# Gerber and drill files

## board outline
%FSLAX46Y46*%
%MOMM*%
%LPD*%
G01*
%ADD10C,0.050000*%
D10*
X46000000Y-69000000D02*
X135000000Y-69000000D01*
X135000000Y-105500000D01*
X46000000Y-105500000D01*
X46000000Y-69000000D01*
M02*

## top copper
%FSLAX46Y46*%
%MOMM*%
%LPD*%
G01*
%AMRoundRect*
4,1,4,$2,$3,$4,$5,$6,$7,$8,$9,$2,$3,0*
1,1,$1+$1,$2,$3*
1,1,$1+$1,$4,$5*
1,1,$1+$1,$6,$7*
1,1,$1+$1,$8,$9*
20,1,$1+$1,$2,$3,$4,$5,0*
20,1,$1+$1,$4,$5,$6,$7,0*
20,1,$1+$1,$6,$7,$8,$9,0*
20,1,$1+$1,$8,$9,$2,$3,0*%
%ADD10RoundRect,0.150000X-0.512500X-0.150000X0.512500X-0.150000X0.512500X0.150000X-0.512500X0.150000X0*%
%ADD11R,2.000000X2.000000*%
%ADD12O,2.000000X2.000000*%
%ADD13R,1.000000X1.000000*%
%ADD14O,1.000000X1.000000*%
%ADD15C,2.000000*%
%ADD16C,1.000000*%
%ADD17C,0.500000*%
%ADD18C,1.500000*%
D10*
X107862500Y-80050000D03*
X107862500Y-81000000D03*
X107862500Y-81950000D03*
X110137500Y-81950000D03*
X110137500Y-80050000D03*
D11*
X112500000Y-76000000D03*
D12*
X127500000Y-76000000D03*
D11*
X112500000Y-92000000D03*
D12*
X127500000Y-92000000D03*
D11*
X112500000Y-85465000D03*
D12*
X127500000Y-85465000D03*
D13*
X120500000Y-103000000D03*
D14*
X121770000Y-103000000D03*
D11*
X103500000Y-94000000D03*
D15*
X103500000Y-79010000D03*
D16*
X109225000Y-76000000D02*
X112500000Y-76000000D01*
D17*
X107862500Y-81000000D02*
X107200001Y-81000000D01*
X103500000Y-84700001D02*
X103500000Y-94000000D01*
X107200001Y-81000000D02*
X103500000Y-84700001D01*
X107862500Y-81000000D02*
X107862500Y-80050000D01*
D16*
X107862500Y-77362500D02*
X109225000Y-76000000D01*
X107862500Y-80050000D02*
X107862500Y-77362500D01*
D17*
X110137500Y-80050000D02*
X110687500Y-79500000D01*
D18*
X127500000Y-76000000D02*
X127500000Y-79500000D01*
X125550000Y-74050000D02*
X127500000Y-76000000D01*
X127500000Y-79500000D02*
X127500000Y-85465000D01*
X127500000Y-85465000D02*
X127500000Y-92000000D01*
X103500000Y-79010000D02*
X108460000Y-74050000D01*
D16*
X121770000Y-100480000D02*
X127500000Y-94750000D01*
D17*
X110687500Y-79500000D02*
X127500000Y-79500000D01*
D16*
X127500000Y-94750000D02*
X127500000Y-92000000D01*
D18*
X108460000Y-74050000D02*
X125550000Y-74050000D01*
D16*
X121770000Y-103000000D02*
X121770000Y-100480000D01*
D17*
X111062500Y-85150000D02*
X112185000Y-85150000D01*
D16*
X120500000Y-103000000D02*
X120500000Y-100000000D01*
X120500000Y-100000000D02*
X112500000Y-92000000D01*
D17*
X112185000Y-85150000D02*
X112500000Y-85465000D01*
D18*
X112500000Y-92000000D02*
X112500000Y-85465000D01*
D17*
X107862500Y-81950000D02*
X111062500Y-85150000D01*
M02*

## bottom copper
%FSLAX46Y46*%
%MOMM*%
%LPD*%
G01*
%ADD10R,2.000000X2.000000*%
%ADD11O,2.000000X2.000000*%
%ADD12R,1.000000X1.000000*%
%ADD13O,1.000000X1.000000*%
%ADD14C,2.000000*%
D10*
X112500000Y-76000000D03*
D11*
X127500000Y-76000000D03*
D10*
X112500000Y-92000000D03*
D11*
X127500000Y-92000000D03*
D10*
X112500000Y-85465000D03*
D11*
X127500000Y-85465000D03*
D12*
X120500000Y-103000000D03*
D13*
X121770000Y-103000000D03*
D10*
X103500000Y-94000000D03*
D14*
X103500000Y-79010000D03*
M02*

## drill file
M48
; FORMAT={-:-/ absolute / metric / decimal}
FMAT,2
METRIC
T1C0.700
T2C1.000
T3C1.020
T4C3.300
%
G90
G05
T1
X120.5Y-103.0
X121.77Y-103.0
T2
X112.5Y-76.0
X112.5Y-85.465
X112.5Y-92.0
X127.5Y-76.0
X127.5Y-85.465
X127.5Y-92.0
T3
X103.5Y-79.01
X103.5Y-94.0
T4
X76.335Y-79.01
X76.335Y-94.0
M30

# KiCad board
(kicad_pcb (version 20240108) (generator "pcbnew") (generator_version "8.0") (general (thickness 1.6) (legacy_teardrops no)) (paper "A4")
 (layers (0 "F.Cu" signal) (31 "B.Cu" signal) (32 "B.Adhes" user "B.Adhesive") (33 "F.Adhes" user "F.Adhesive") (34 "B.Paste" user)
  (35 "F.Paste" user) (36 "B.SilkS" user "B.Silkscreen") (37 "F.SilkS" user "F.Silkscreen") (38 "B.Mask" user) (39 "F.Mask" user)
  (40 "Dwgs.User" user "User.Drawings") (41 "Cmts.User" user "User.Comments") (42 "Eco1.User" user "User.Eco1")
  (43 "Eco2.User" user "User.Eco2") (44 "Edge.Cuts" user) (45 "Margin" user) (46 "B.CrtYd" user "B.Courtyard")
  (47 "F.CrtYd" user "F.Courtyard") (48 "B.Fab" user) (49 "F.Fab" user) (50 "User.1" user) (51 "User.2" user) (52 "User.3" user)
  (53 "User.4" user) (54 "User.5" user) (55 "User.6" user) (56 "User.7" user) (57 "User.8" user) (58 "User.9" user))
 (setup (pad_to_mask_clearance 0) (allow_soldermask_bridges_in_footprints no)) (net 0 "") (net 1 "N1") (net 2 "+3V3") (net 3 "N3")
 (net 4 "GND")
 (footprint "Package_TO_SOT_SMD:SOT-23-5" (layer "F.Cu") (at 109 81)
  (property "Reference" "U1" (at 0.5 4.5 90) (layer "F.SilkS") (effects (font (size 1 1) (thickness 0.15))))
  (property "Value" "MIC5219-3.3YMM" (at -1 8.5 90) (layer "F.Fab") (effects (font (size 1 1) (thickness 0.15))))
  (pad "1" smd roundrect (at -1.1375 -0.95) (size 1.325 0.6) (layers "F.Cu" "F.Paste" "F.Mask") (roundrect_rratio 0.25) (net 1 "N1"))
  (pad "2" smd roundrect (at -1.1375 0) (size 1.325 0.6) (layers "F.Cu" "F.Paste" "F.Mask") (roundrect_rratio 0.25) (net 1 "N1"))
  (pad "3" smd roundrect (at -1.1375 0.95) (size 1.325 0.6) (layers "F.Cu" "F.Paste" "F.Mask") (roundrect_rratio 0.25) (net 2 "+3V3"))
  (pad "4" smd roundrect (at 1.1375 0.95) (size 1.325 0.6) (layers "F.Cu" "F.Paste" "F.Mask") (roundrect_rratio 0.25) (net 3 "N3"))
  (pad "5" smd roundrect (at 1.1375 -0.95) (size 1.325 0.6) (layers "F.Cu" "F.Paste" "F.Mask") (roundrect_rratio 0.25) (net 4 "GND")))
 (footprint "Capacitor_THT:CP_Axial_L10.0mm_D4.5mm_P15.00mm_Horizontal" (layer "F.Cu") (at 112.5 76)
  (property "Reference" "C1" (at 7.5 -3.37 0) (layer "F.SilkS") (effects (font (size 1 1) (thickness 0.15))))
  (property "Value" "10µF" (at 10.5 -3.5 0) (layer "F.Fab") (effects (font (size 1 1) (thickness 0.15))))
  (pad "1" thru_hole rect (at 0 0) (size 2 2) (drill 1) (layers "*.Cu" "*.Mask") (remove_unused_layers no) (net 1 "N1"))
  (pad "2" thru_hole oval (at 15 0) (size 2 2) (drill 1) (layers "*.Cu" "*.Mask") (remove_unused_layers no) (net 4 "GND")))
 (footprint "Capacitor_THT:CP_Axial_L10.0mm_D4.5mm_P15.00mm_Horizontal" (layer "F.Cu") (at 112.5 92)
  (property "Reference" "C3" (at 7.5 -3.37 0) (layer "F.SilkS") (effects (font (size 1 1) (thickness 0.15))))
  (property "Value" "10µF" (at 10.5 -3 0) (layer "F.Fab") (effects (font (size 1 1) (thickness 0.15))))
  (pad "1" thru_hole rect (at 0 0) (size 2 2) (drill 1) (layers "*.Cu" "*.Mask") (remove_unused_layers no) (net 2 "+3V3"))
  (pad "2" thru_hole oval (at 15 0) (size 2 2) (drill 1) (layers "*.Cu" "*.Mask") (remove_unused_layers no) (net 4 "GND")))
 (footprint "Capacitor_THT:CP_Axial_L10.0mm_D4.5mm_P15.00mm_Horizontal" (layer "F.Cu") (at 112.5 85.465)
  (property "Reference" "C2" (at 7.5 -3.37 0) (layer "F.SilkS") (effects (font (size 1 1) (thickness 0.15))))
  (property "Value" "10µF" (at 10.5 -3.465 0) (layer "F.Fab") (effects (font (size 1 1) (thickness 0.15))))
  (pad "1" thru_hole rect (at 0 0) (size 2 2) (drill 1) (layers "*.Cu" "*.Mask") (remove_unused_layers no) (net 2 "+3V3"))
  (pad "2" thru_hole oval (at 15 0) (size 2 2) (drill 1) (layers "*.Cu" "*.Mask") (remove_unused_layers no) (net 4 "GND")))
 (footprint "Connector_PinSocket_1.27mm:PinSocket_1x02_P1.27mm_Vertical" (layer "F.Cu") (at 120.5 103 90)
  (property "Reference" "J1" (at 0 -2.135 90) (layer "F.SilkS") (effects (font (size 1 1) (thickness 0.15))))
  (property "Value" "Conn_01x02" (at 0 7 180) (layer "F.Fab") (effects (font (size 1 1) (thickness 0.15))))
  (pad "1" thru_hole rect (at 0 0 90) (size 1 1) (drill 0.7) (layers "*.Cu" "*.Mask") (remove_unused_layers no) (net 2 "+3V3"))
  (pad "2" thru_hole oval (at 0 1.27 90) (size 1 1) (drill 0.7) (layers "*.Cu" "*.Mask") (remove_unused_layers no) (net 4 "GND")))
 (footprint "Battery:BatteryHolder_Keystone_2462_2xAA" (layer "F.Cu") (at 103.5 94 180)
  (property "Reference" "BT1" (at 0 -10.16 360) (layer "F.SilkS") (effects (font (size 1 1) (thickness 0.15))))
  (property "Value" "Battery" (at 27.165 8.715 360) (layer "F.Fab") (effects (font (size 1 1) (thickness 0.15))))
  (pad "" np_thru_hole circle (at 27.165 0 180) (size 3.3 3.3) (drill 3.3) (layers "*.Cu" "*.Mask"))
  (pad "" np_thru_hole circle (at 27.165 14.99 180) (size 3.3 3.3) (drill 3.3) (layers "*.Cu" "*.Mask"))
  (pad "1" thru_hole rect (at 0 0 180) (size 2 2) (drill 1.02) (layers "*.Cu" "*.Mask") (remove_unused_layers no) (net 1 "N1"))
  (pad "2" thru_hole circle (at 0 14.99 180) (size 2 2) (drill 1.02) (layers "*.Cu" "*.Mask") (remove_unused_layers no) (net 4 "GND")))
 (gr_rect (start 46 69) (end 135 105.5) (stroke (width 0.05) (type default)) (fill none) (layer "Edge.Cuts"))
 (segment (start 109.225 76) (end 112.5 76) (width 1) (layer "F.Cu") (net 1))
 (segment (start 107.8625 81) (end 107.200001 81) (width 0.5) (layer "F.Cu") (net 1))
 (segment (start 103.5 84.700001) (end 103.5 94) (width 0.5) (layer "F.Cu") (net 1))
 (segment (start 107.200001 81) (end 103.5 84.700001) (width 0.5) (layer "F.Cu") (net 1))
 (segment (start 107.8625 81) (end 107.8625 80.05) (width 0.5) (layer "F.Cu") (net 1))
 (segment (start 107.8625 77.3625) (end 109.225 76) (width 1) (layer "F.Cu") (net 1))
 (segment (start 107.8625 80.05) (end 107.8625 77.3625) (width 1) (layer "F.Cu") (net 1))
 (segment (start 110.1375 80.05) (end 110.6875 79.5) (width 0.5) (layer "F.Cu") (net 4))
 (segment (start 127.5 76) (end 127.5 79.5) (width 1.5) (layer "F.Cu") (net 4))
 (segment (start 125.55 74.05) (end 127.5 76) (width 1.5) (layer "F.Cu") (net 4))
 (segment (start 127.5 79.5) (end 127.5 85.465) (width 1.5) (layer "F.Cu") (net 4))
 (segment (start 127.5 85.465) (end 127.5 92) (width 1.5) (layer "F.Cu") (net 4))
 (segment (start 103.5 79.01) (end 108.46 74.05) (width 1.5) (layer "F.Cu") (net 4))
 (segment (start 121.77 100.48) (end 127.5 94.75) (width 1) (layer "F.Cu") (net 4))
 (segment (start 110.6875 79.5) (end 127.5 79.5) (width 0.5) (layer "F.Cu") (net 4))
 (segment (start 127.5 94.75) (end 127.5 92) (width 1) (layer "F.Cu") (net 4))
 (segment (start 108.46 74.05) (end 125.55 74.05) (width 1.5) (layer "F.Cu") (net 4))
 (segment (start 121.77 103) (end 121.77 100.48) (width 1) (layer "F.Cu") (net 4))
 (segment (start 111.0625 85.15) (end 112.185 85.15) (width 0.5) (layer "F.Cu") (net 2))
 (segment (start 120.5 103) (end 120.5 100) (width 1) (layer "F.Cu") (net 2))
 (segment (start 120.5 100) (end 112.5 92) (width 1) (layer "F.Cu") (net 2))
 (segment (start 112.185 85.15) (end 112.5 85.465) (width 0.5) (layer "F.Cu") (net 2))
 (segment (start 112.5 92) (end 112.5 85.465) (width 1.5) (layer "F.Cu") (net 2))
 (segment (start 107.8625 81.95) (end 111.0625 85.15) (width 0.5) (layer "F.Cu") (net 2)))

